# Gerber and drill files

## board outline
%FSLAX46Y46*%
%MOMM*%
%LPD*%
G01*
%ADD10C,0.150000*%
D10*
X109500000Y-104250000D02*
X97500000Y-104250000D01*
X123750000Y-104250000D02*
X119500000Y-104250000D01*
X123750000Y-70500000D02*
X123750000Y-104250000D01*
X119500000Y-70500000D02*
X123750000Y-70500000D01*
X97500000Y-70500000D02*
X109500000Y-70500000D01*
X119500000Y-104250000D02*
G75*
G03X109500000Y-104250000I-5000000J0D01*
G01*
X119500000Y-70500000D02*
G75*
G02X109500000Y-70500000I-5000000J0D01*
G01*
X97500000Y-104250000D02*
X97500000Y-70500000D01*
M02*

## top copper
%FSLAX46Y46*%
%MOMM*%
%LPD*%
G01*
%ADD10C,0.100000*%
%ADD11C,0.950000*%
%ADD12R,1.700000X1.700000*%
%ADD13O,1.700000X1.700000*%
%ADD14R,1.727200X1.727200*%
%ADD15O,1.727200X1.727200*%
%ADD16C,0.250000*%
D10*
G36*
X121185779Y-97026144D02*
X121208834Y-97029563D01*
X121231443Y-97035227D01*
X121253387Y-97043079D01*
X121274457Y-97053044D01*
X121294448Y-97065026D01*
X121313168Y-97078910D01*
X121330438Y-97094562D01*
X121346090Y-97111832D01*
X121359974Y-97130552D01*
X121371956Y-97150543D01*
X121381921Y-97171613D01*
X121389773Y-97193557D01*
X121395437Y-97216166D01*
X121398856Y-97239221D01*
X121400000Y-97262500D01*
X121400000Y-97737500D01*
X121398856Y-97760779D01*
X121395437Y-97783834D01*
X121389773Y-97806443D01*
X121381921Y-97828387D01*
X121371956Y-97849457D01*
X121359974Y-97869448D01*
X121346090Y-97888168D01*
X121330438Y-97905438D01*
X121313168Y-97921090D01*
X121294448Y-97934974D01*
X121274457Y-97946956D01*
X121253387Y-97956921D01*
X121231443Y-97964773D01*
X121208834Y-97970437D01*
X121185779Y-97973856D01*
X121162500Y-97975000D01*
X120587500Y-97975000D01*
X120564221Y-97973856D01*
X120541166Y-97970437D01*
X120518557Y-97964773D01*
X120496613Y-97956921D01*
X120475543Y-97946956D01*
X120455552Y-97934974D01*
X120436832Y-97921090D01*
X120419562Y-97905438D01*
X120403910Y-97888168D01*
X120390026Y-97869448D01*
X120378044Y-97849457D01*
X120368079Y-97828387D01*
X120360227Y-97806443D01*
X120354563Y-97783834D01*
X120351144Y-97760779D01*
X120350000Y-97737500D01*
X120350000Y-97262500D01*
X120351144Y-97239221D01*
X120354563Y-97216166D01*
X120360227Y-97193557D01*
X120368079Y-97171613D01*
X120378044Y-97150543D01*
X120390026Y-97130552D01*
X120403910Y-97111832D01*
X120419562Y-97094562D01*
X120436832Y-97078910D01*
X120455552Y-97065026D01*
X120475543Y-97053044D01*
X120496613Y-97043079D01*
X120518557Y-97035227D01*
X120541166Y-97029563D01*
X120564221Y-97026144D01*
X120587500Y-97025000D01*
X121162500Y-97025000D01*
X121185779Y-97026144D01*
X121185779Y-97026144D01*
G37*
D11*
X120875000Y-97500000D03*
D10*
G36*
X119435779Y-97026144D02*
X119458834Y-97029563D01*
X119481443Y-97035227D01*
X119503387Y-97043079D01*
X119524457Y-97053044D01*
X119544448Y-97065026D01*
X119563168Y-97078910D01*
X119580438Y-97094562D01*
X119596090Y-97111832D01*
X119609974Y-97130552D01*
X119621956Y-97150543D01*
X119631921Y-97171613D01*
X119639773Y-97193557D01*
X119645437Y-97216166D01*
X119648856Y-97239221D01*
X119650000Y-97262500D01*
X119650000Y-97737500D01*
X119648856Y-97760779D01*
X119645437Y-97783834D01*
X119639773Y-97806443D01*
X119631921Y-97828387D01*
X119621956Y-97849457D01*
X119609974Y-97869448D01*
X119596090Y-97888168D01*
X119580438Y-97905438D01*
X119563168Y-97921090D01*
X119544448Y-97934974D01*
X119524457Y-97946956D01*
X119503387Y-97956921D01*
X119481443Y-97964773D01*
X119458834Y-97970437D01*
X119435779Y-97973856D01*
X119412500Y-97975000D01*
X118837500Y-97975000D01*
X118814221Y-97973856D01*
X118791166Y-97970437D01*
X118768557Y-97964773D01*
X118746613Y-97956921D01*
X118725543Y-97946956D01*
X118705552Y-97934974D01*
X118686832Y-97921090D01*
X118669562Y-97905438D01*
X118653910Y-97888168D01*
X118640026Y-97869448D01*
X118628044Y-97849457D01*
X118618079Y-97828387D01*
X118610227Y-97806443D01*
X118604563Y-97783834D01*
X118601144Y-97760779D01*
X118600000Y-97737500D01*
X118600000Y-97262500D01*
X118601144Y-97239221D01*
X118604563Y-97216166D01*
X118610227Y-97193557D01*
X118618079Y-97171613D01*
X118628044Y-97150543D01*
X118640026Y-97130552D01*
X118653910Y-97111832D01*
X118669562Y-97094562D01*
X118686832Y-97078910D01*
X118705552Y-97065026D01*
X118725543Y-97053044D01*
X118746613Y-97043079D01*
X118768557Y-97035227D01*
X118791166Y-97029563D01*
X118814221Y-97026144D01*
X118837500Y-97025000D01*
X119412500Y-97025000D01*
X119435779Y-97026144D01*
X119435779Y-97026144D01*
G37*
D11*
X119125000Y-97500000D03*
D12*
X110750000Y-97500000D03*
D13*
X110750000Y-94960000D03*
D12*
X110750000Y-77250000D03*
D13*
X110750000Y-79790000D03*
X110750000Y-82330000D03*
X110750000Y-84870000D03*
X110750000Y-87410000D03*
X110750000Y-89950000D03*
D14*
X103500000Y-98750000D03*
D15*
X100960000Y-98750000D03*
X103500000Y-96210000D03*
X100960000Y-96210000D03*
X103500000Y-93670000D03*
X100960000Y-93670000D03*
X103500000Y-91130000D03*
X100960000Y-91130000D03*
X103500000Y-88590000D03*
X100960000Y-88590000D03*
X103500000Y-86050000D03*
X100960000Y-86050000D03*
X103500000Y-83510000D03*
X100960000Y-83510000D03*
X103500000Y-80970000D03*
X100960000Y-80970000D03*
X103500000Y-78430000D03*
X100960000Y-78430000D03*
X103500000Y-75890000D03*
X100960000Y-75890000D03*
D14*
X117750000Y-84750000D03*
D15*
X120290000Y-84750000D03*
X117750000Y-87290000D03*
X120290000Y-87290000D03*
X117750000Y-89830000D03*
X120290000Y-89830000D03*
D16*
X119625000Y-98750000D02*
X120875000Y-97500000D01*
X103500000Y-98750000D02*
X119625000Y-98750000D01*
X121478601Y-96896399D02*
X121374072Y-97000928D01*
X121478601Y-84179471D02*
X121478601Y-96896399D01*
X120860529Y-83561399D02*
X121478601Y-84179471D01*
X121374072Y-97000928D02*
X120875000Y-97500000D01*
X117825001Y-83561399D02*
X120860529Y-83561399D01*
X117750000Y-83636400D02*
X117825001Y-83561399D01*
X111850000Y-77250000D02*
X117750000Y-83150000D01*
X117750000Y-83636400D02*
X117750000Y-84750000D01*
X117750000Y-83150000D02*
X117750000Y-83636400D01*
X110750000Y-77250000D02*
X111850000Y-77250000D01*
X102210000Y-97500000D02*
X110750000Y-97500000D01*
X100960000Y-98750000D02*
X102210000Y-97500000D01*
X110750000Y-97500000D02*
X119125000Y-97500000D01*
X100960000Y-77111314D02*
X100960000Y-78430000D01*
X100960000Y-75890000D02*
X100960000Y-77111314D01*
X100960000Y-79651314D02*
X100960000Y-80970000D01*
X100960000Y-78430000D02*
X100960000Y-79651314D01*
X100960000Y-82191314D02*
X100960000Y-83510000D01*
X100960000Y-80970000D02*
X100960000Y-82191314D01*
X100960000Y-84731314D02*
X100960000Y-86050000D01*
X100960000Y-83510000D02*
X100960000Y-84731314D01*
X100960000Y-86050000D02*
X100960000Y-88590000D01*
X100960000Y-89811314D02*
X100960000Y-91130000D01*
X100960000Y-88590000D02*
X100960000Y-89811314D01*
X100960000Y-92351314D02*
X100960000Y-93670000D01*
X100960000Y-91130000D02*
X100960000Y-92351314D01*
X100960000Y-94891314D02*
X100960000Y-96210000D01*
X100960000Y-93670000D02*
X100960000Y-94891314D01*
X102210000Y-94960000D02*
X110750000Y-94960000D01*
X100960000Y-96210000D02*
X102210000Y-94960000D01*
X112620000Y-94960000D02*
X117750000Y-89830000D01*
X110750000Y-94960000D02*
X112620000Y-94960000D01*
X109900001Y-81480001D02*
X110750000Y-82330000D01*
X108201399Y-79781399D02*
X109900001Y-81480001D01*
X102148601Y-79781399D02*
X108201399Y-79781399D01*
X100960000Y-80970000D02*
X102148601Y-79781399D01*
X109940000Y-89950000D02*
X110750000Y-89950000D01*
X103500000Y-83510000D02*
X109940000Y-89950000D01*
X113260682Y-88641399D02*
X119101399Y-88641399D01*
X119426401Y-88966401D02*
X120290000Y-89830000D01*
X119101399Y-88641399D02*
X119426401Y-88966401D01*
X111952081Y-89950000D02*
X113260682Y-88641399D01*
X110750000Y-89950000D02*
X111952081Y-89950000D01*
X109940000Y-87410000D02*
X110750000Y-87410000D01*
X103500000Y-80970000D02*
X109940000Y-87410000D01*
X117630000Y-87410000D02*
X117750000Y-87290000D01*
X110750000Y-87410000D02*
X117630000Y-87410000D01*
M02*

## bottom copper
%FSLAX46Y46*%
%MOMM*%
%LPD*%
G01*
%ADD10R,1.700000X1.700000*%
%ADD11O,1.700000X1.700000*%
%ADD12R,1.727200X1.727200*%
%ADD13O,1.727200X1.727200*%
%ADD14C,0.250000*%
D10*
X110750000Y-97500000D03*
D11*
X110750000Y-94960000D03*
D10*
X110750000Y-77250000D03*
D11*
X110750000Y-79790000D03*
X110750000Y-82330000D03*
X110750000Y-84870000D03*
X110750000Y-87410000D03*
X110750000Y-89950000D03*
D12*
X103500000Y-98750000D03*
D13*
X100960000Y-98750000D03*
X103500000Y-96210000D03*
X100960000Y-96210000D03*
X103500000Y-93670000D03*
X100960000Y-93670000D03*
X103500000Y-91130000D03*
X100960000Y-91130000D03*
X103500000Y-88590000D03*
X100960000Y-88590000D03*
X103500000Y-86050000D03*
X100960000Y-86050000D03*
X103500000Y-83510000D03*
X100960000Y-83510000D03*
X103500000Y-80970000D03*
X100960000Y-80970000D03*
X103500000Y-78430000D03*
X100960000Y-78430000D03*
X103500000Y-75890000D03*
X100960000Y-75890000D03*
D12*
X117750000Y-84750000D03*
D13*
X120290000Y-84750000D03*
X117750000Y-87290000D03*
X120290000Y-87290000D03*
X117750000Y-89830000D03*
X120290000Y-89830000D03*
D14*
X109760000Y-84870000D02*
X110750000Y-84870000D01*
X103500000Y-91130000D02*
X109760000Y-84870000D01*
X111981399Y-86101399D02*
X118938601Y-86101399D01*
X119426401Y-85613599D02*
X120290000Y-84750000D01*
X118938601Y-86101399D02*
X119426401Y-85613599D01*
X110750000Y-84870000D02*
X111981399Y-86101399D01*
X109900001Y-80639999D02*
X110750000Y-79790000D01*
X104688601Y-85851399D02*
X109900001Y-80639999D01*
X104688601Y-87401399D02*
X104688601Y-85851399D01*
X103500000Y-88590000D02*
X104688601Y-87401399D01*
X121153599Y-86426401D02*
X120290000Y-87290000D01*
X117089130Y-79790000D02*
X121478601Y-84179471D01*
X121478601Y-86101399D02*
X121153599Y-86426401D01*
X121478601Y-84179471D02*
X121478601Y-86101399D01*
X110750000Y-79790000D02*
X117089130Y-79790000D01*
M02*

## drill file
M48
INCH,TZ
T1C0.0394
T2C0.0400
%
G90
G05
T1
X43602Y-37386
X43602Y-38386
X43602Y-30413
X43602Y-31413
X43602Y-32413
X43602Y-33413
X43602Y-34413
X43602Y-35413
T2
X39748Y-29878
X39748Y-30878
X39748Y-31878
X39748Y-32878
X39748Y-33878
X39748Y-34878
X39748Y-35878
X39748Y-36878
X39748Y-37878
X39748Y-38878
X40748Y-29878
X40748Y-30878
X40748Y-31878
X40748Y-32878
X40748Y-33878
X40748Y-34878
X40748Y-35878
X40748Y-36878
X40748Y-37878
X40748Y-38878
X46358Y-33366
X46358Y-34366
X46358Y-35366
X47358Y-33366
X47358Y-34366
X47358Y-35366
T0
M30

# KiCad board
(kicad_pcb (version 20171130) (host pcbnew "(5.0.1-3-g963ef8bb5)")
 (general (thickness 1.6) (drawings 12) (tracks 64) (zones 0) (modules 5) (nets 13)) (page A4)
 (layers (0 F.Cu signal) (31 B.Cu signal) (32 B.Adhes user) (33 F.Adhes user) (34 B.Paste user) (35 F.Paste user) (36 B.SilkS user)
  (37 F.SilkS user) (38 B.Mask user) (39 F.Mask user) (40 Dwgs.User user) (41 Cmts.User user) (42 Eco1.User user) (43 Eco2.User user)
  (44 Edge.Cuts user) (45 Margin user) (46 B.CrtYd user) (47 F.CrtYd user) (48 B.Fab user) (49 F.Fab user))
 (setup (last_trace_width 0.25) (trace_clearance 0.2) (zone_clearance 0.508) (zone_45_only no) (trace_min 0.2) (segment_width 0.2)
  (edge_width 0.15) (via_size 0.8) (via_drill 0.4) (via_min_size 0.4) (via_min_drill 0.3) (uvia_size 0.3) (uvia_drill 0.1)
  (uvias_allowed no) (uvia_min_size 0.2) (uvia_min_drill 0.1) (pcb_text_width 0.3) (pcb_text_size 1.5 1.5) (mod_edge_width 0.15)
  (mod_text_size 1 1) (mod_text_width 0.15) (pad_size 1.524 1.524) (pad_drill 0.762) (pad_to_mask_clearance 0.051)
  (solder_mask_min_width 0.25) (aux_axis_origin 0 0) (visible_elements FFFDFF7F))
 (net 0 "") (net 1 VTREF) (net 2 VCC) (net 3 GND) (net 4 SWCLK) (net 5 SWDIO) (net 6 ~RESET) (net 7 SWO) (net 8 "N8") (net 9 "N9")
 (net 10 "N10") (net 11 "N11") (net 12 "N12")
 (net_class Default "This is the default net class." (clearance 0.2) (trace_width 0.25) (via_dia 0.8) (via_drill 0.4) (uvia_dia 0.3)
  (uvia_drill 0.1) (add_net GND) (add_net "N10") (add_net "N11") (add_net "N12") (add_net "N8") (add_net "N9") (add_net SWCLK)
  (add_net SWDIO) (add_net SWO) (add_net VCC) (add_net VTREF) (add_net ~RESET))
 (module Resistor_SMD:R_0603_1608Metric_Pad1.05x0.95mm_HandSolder (layer F.Cu) (at 120 97.5 180)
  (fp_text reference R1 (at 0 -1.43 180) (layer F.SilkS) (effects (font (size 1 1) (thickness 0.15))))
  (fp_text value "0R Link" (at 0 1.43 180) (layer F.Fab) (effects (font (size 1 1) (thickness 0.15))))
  (pad 1 smd roundrect (at -0.875 0 180) (size 1.05 0.95) (layers F.Cu F.Paste F.Mask) (roundrect_rratio 0.25) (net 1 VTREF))
  (pad 2 smd roundrect (at 0.875 0 180) (size 1.05 0.95) (layers F.Cu F.Paste F.Mask) (roundrect_rratio 0.25) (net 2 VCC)))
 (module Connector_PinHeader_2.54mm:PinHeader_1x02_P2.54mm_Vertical (layer F.Cu) (at 110.75 97.5 180)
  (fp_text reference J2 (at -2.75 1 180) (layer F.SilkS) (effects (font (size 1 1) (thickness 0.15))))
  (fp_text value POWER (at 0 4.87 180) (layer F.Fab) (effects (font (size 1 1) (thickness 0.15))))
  (pad 1 thru_hole rect (at 0 0 180) (size 1.7 1.7) (drill 1) (layers *.Cu *.Mask) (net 2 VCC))
  (pad 2 thru_hole oval (at 0 2.54 180) (size 1.7 1.7) (drill 1) (layers *.Cu *.Mask) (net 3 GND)))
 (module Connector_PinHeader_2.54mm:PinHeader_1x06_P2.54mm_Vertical (layer F.Cu) (at 110.75 77.25)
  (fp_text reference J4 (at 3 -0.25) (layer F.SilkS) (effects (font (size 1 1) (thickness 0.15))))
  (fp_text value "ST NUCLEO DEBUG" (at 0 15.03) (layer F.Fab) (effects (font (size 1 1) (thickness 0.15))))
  (pad 1 thru_hole rect (at 0 0) (size 1.7 1.7) (drill 1) (layers *.Cu *.Mask) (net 1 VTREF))
  (pad 2 thru_hole oval (at 0 2.54) (size 1.7 1.7) (drill 1) (layers *.Cu *.Mask) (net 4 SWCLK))
  (pad 3 thru_hole oval (at 0 5.08) (size 1.7 1.7) (drill 1) (layers *.Cu *.Mask) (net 3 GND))
  (pad 4 thru_hole oval (at 0 7.62) (size 1.7 1.7) (drill 1) (layers *.Cu *.Mask) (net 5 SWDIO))
  (pad 5 thru_hole oval (at 0 10.16) (size 1.7 1.7) (drill 1) (layers *.Cu *.Mask) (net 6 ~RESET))
  (pad 6 thru_hole oval (at 0 12.7) (size 1.7 1.7) (drill 1) (layers *.Cu *.Mask) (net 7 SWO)))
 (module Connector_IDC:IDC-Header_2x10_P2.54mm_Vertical (layer F.Cu) (at 103.5 98.75 180)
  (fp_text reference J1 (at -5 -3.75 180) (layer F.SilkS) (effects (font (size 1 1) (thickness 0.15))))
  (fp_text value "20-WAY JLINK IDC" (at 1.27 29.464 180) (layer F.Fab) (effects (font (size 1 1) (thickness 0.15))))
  (pad 1 thru_hole rect (at 0 0 180) (size 1.7272 1.7272) (drill 1.016) (layers *.Cu *.Mask) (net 1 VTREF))
  (pad 2 thru_hole oval (at 2.54 0 180) (size 1.7272 1.7272) (drill 1.016) (layers *.Cu *.Mask) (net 2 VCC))
  (pad 3 thru_hole oval (at 0 2.54 180) (size 1.7272 1.7272) (drill 1.016) (layers *.Cu *.Mask) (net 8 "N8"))
  (pad 4 thru_hole oval (at 2.54 2.54 180) (size 1.7272 1.7272) (drill 1.016) (layers *.Cu *.Mask) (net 3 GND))
  (pad 5 thru_hole oval (at 0 5.08 180) (size 1.7272 1.7272) (drill 1.016) (layers *.Cu *.Mask) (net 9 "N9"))
  (pad 6 thru_hole oval (at 2.54 5.08 180) (size 1.7272 1.7272) (drill 1.016) (layers *.Cu *.Mask) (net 3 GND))
  (pad 7 thru_hole oval (at 0 7.62 180) (size 1.7272 1.7272) (drill 1.016) (layers *.Cu *.Mask) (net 5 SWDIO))
  (pad 8 thru_hole oval (at 2.54 7.62 180) (size 1.7272 1.7272) (drill 1.016) (layers *.Cu *.Mask) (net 3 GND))
  (pad 9 thru_hole oval (at 0 10.16 180) (size 1.7272 1.7272) (drill 1.016) (layers *.Cu *.Mask) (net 4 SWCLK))
  (pad 10 thru_hole oval (at 2.54 10.16 180) (size 1.7272 1.7272) (drill 1.016) (layers *.Cu *.Mask) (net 3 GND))
  (pad 11 thru_hole oval (at 0 12.7 180) (size 1.7272 1.7272) (drill 1.016) (layers *.Cu *.Mask) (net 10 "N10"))
  (pad 12 thru_hole oval (at 2.54 12.7 180) (size 1.7272 1.7272) (drill 1.016) (layers *.Cu *.Mask) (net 3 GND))
  (pad 13 thru_hole oval (at 0 15.24 180) (size 1.7272 1.7272) (drill 1.016) (layers *.Cu *.Mask) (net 7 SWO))
  (pad 14 thru_hole oval (at 2.54 15.24 180) (size 1.7272 1.7272) (drill 1.016) (layers *.Cu *.Mask) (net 3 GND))
  (pad 15 thru_hole oval (at 0 17.78 180) (size 1.7272 1.7272) (drill 1.016) (layers *.Cu *.Mask) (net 6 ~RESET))
  (pad 16 thru_hole oval (at 2.54 17.78 180) (size 1.7272 1.7272) (drill 1.016) (layers *.Cu *.Mask) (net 3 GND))
  (pad 17 thru_hole oval (at 0 20.32 180) (size 1.7272 1.7272) (drill 1.016) (layers *.Cu *.Mask) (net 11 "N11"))
  (pad 18 thru_hole oval (at 2.54 20.32 180) (size 1.7272 1.7272) (drill 1.016) (layers *.Cu *.Mask) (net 3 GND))
  (pad 19 thru_hole oval (at 0 22.86 180) (size 1.7272 1.7272) (drill 1.016) (layers *.Cu *.Mask) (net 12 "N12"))
  (pad 20 thru_hole oval (at 2.54 22.86 180) (size 1.7272 1.7272) (drill 1.016) (layers *.Cu *.Mask) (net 3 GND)))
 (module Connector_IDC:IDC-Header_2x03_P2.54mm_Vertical (layer F.Cu) (at 117.75 84.75)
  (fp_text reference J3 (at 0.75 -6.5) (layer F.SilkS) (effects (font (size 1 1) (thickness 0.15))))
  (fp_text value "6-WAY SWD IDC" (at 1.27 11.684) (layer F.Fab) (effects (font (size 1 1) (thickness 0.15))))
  (pad 1 thru_hole rect (at 0 0) (size 1.7272 1.7272) (drill 1.016) (layers *.Cu *.Mask) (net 1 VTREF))
  (pad 2 thru_hole oval (at 2.54 0) (size 1.7272 1.7272) (drill 1.016) (layers *.Cu *.Mask) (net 5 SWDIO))
  (pad 3 thru_hole oval (at 0 2.54) (size 1.7272 1.7272) (drill 1.016) (layers *.Cu *.Mask) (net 6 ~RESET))
  (pad 4 thru_hole oval (at 2.54 2.54) (size 1.7272 1.7272) (drill 1.016) (layers *.Cu *.Mask) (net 4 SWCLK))
  (pad 5 thru_hole oval (at 0 5.08) (size 1.7272 1.7272) (drill 1.016) (layers *.Cu *.Mask) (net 3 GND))
  (pad 6 thru_hole oval (at 2.54 5.08) (size 1.7272 1.7272) (drill 1.016) (layers *.Cu *.Mask) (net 7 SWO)))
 (gr_line (start 109.5 104.25) (end 97.5 104.25) (layer Edge.Cuts) (width 0.15))
 (gr_line (start 123.75 104.25) (end 119.5 104.25) (layer Edge.Cuts) (width 0.15))
 (gr_line (start 123.75 70.5) (end 123.75 104.25) (layer Edge.Cuts) (width 0.15))
 (gr_line (start 119.5 70.5) (end 123.75 70.5) (layer Edge.Cuts) (width 0.15))
 (gr_line (start 97.5 70.5) (end 109.5 70.5) (layer Edge.Cuts) (width 0.15))
 (gr_arc (start 114.5 104.25) (end 109.5 104.25) (angle 180) (layer Edge.Cuts) (width 0.15))
 (gr_arc (start 114.5 70.5) (end 109.5 70.5) (angle -180) (layer Edge.Cuts) (width 0.15))
 (gr_line (start 97.5 104.25) (end 97.5 70.5) (layer Edge.Cuts) (width 0.15))
 (segment (start 119.625 98.75) (end 120.875 97.5) (width 0.25) (layer F.Cu) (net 1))
 (segment (start 103.5 98.75) (end 119.625 98.75) (width 0.25) (layer F.Cu) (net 1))
 (segment (start 121.478601 96.896399) (end 121.374072 97.000928) (width 0.25) (layer F.Cu) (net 1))
 (segment (start 121.478601 84.179471) (end 121.478601 96.896399) (width 0.25) (layer F.Cu) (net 1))
 (segment (start 120.860529 83.561399) (end 121.478601 84.179471) (width 0.25) (layer F.Cu) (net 1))
 (segment (start 121.374072 97.000928) (end 120.875 97.5) (width 0.25) (layer F.Cu) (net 1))
 (segment (start 117.825001 83.561399) (end 120.860529 83.561399) (width 0.25) (layer F.Cu) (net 1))
 (segment (start 117.75 83.6364) (end 117.825001 83.561399) (width 0.25) (layer F.Cu) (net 1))
 (segment (start 111.85 77.25) (end 117.75 83.15) (width 0.25) (layer F.Cu) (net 1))
 (segment (start 117.75 83.6364) (end 117.75 84.75) (width 0.25) (layer F.Cu) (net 1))
 (segment (start 117.75 83.15) (end 117.75 83.6364) (width 0.25) (layer F.Cu) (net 1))
 (segment (start 110.75 77.25) (end 111.85 77.25) (width 0.25) (layer F.Cu) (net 1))
 (segment (start 102.21 97.5) (end 110.75 97.5) (width 0.25) (layer F.Cu) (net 2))
 (segment (start 100.96 98.75) (end 102.21 97.5) (width 0.25) (layer F.Cu) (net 2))
 (segment (start 110.75 97.5) (end 119.125 97.5) (width 0.25) (layer F.Cu) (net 2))
 (segment (start 100.96 77.111314) (end 100.96 78.43) (width 0.25) (layer F.Cu) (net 3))
 (segment (start 100.96 75.89) (end 100.96 77.111314) (width 0.25) (layer F.Cu) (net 3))
 (segment (start 100.96 79.651314) (end 100.96 80.97) (width 0.25) (layer F.Cu) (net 3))
 (segment (start 100.96 78.43) (end 100.96 79.651314) (width 0.25) (layer F.Cu) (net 3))
 (segment (start 100.96 82.191314) (end 100.96 83.51) (width 0.25) (layer F.Cu) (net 3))
 (segment (start 100.96 80.97) (end 100.96 82.191314) (width 0.25) (layer F.Cu) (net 3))
 (segment (start 100.96 84.731314) (end 100.96 86.05) (width 0.25) (layer F.Cu) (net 3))
 (segment (start 100.96 83.51) (end 100.96 84.731314) (width 0.25) (layer F.Cu) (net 3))
 (segment (start 100.96 86.05) (end 100.96 88.59) (width 0.25) (layer F.Cu) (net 3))
 (segment (start 100.96 89.811314) (end 100.96 91.13) (width 0.25) (layer F.Cu) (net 3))
 (segment (start 100.96 88.59) (end 100.96 89.811314) (width 0.25) (layer F.Cu) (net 3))
 (segment (start 100.96 92.351314) (end 100.96 93.67) (width 0.25) (layer F.Cu) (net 3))
 (segment (start 100.96 91.13) (end 100.96 92.351314) (width 0.25) (layer F.Cu) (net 3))
 (segment (start 100.96 94.891314) (end 100.96 96.21) (width 0.25) (layer F.Cu) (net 3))
 (segment (start 100.96 93.67) (end 100.96 94.891314) (width 0.25) (layer F.Cu) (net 3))
 (segment (start 102.21 94.96) (end 110.75 94.96) (width 0.25) (layer F.Cu) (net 3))
 (segment (start 100.96 96.21) (end 102.21 94.96) (width 0.25) (layer F.Cu) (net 3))
 (segment (start 112.62 94.96) (end 117.75 89.83) (width 0.25) (layer F.Cu) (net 3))
 (segment (start 110.75 94.96) (end 112.62 94.96) (width 0.25) (layer F.Cu) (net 3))
 (segment (start 109.900001 81.480001) (end 110.75 82.33) (width 0.25) (layer F.Cu) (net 3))
 (segment (start 108.201399 79.781399) (end 109.900001 81.480001) (width 0.25) (layer F.Cu) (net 3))
 (segment (start 102.148601 79.781399) (end 108.201399 79.781399) (width 0.25) (layer F.Cu) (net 3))
 (segment (start 100.96 80.97) (end 102.148601 79.781399) (width 0.25) (layer F.Cu) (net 3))
 (segment (start 109.76 84.87) (end 110.75 84.87) (width 0.25) (layer B.Cu) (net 5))
 (segment (start 103.5 91.13) (end 109.76 84.87) (width 0.25) (layer B.Cu) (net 5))
 (segment (start 111.981399 86.101399) (end 118.938601 86.101399) (width 0.25) (layer B.Cu) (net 5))
 (segment (start 119.426401 85.613599) (end 120.29 84.75) (width 0.25) (layer B.Cu) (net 5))
 (segment (start 118.938601 86.101399) (end 119.426401 85.613599) (width 0.25) (layer B.Cu) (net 5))
 (segment (start 110.75 84.87) (end 111.981399 86.101399) (width 0.25) (layer B.Cu) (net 5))
 (segment (start 109.900001 80.639999) (end 110.75 79.79) (width 0.25) (layer B.Cu) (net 4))
 (segment (start 104.688601 85.851399) (end 109.900001 80.639999) (width 0.25) (layer B.Cu) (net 4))
 (segment (start 104.688601 87.401399) (end 104.688601 85.851399) (width 0.25) (layer B.Cu) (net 4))
 (segment (start 103.5 88.59) (end 104.688601 87.401399) (width 0.25) (layer B.Cu) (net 4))
 (segment (start 121.153599 86.426401) (end 120.29 87.29) (width 0.25) (layer B.Cu) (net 4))
 (segment (start 117.08913 79.79) (end 121.478601 84.179471) (width 0.25) (layer B.Cu) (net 4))
 (segment (start 121.478601 86.101399) (end 121.153599 86.426401) (width 0.25) (layer B.Cu) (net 4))
 (segment (start 121.478601 84.179471) (end 121.478601 86.101399) (width 0.25) (layer B.Cu) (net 4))
 (segment (start 110.75 79.79) (end 117.08913 79.79) (width 0.25) (layer B.Cu) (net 4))
 (segment (start 109.94 89.95) (end 110.75 89.95) (width 0.25) (layer F.Cu) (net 7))
 (segment (start 103.5 83.51) (end 109.94 89.95) (width 0.25) (layer F.Cu) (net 7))
 (segment (start 113.260682 88.641399) (end 119.101399 88.641399) (width 0.25) (layer F.Cu) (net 7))
 (segment (start 119.426401 88.966401) (end 120.29 89.83) (width 0.25) (layer F.Cu) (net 7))
 (segment (start 119.101399 88.641399) (end 119.426401 88.966401) (width 0.25) (layer F.Cu) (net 7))
 (segment (start 111.952081 89.95) (end 113.260682 88.641399) (width 0.25) (layer F.Cu) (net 7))
 (segment (start 110.75 89.95) (end 111.952081 89.95) (width 0.25) (layer F.Cu) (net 7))
 (segment (start 109.94 87.41) (end 110.75 87.41) (width 0.25) (layer F.Cu) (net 6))
 (segment (start 103.5 80.97) (end 109.94 87.41) (width 0.25) (layer F.Cu) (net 6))
 (segment (start 117.63 87.41) (end 117.75 87.29) (width 0.25) (layer F.Cu) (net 6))
 (segment (start 110.75 87.41) (end 117.63 87.41) (width 0.25) (layer F.Cu) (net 6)))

